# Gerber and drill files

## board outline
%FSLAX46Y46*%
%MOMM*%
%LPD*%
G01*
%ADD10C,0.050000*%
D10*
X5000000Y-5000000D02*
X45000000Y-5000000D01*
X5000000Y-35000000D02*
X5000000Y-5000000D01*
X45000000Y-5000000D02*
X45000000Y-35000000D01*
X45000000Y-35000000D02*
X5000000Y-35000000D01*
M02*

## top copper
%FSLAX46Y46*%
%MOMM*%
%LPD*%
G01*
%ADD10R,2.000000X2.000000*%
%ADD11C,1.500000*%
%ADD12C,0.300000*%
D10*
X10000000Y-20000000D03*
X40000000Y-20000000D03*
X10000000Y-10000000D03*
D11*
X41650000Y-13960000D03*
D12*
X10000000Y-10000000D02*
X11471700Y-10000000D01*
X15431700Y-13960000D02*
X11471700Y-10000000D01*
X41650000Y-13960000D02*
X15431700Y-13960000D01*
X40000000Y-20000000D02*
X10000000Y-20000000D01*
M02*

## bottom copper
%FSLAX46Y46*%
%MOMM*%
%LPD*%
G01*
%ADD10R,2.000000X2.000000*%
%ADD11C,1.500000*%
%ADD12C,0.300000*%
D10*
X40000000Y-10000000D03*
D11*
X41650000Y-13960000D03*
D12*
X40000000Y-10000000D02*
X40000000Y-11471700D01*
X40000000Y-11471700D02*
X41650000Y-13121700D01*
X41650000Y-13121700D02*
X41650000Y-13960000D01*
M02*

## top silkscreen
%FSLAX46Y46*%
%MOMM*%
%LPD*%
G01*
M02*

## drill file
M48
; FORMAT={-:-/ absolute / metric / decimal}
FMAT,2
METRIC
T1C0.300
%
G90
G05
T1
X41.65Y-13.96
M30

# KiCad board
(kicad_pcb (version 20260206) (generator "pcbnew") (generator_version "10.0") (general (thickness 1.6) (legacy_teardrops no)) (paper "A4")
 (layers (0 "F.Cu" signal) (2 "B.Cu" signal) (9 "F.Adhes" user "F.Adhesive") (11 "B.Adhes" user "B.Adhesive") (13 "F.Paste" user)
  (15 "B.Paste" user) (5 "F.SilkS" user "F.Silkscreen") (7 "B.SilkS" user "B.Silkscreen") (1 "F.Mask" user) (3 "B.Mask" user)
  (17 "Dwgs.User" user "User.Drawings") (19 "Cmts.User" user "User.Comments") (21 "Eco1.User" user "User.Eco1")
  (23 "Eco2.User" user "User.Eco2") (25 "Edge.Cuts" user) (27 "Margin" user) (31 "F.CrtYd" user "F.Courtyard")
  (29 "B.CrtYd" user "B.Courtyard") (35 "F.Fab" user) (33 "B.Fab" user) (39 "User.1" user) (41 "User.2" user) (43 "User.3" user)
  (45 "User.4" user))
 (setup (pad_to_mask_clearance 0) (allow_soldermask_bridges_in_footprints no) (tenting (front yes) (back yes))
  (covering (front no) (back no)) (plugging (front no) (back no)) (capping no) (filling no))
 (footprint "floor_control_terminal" (layer "F.Cu") (at 10 20)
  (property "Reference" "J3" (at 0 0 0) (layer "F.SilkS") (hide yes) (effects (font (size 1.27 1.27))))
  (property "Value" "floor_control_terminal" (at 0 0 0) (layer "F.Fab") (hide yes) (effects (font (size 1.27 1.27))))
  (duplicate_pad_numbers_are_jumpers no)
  (pad "1" smd rect (at 0 0) (size 2 2) (layers "F.Cu" "F.Mask" "F.Paste") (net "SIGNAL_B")))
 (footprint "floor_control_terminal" (layer "F.Cu") (at 40 20)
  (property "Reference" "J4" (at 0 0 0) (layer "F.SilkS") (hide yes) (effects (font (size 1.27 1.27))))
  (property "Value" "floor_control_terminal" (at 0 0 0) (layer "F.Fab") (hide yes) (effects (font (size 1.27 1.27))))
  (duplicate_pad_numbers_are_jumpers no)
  (pad "1" smd rect (at 0 0) (size 2 2) (layers "F.Cu" "F.Mask" "F.Paste") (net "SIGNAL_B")))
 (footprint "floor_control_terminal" (layer "F.Cu") (at 10 10)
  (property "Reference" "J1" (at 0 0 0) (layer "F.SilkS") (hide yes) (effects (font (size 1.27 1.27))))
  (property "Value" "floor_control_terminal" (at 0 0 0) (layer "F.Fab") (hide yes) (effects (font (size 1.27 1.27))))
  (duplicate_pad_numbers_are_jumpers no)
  (pad "1" smd rect (at 0 0) (size 2 2) (layers "F.Cu" "F.Mask" "F.Paste") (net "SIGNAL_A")))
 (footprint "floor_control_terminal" (layer "B.Cu") (at 40 10)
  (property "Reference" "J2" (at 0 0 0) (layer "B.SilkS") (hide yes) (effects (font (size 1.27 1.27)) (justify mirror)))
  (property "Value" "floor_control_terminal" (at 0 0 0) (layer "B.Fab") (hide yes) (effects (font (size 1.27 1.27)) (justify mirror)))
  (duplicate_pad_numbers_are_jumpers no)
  (pad "1" smd rect (at 0 0) (size 2 2) (layers "B.Cu" "B.Mask" "B.Paste") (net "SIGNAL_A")))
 (gr_line (start 5 5) (end 45 5) (stroke (width 0.05) (type default)) (layer "Edge.Cuts"))
 (gr_line (start 5 35) (end 5 5) (stroke (width 0.05) (type default)) (layer "Edge.Cuts"))
 (gr_line (start 45 5) (end 45 35) (stroke (width 0.05) (type default)) (layer "Edge.Cuts"))
 (gr_line (start 45 35) (end 5 35) (stroke (width 0.05) (type default)) (layer "Edge.Cuts"))
 (segment (start 10 10) (end 11.4717 10) (width 0.3) (layer "F.Cu") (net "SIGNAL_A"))
 (segment (start 15.4317 13.96) (end 11.4717 10) (width 0.3) (layer "F.Cu") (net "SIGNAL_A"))
 (segment (start 41.65 13.96) (end 15.4317 13.96) (width 0.3) (layer "F.Cu") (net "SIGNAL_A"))
 (via (at 41.65 13.96) (size 1.5) (drill 0.3) (layers "F.Cu" "B.Cu") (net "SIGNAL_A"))
 (segment (start 40 10) (end 40 11.4717) (width 0.3) (layer "B.Cu") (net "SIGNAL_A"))
 (segment (start 40 11.4717) (end 41.65 13.1217) (width 0.3) (layer "B.Cu") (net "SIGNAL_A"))
 (segment (start 41.65 13.1217) (end 41.65 13.96) (width 0.3) (layer "B.Cu") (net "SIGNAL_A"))
 (segment (start 40 20) (end 10 20) (width 0.3) (layer "F.Cu") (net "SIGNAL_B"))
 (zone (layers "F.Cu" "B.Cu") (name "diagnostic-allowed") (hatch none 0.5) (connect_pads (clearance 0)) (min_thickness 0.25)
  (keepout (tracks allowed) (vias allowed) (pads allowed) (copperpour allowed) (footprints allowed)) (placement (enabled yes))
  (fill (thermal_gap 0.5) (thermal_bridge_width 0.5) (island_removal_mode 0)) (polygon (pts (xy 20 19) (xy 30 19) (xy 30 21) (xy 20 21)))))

